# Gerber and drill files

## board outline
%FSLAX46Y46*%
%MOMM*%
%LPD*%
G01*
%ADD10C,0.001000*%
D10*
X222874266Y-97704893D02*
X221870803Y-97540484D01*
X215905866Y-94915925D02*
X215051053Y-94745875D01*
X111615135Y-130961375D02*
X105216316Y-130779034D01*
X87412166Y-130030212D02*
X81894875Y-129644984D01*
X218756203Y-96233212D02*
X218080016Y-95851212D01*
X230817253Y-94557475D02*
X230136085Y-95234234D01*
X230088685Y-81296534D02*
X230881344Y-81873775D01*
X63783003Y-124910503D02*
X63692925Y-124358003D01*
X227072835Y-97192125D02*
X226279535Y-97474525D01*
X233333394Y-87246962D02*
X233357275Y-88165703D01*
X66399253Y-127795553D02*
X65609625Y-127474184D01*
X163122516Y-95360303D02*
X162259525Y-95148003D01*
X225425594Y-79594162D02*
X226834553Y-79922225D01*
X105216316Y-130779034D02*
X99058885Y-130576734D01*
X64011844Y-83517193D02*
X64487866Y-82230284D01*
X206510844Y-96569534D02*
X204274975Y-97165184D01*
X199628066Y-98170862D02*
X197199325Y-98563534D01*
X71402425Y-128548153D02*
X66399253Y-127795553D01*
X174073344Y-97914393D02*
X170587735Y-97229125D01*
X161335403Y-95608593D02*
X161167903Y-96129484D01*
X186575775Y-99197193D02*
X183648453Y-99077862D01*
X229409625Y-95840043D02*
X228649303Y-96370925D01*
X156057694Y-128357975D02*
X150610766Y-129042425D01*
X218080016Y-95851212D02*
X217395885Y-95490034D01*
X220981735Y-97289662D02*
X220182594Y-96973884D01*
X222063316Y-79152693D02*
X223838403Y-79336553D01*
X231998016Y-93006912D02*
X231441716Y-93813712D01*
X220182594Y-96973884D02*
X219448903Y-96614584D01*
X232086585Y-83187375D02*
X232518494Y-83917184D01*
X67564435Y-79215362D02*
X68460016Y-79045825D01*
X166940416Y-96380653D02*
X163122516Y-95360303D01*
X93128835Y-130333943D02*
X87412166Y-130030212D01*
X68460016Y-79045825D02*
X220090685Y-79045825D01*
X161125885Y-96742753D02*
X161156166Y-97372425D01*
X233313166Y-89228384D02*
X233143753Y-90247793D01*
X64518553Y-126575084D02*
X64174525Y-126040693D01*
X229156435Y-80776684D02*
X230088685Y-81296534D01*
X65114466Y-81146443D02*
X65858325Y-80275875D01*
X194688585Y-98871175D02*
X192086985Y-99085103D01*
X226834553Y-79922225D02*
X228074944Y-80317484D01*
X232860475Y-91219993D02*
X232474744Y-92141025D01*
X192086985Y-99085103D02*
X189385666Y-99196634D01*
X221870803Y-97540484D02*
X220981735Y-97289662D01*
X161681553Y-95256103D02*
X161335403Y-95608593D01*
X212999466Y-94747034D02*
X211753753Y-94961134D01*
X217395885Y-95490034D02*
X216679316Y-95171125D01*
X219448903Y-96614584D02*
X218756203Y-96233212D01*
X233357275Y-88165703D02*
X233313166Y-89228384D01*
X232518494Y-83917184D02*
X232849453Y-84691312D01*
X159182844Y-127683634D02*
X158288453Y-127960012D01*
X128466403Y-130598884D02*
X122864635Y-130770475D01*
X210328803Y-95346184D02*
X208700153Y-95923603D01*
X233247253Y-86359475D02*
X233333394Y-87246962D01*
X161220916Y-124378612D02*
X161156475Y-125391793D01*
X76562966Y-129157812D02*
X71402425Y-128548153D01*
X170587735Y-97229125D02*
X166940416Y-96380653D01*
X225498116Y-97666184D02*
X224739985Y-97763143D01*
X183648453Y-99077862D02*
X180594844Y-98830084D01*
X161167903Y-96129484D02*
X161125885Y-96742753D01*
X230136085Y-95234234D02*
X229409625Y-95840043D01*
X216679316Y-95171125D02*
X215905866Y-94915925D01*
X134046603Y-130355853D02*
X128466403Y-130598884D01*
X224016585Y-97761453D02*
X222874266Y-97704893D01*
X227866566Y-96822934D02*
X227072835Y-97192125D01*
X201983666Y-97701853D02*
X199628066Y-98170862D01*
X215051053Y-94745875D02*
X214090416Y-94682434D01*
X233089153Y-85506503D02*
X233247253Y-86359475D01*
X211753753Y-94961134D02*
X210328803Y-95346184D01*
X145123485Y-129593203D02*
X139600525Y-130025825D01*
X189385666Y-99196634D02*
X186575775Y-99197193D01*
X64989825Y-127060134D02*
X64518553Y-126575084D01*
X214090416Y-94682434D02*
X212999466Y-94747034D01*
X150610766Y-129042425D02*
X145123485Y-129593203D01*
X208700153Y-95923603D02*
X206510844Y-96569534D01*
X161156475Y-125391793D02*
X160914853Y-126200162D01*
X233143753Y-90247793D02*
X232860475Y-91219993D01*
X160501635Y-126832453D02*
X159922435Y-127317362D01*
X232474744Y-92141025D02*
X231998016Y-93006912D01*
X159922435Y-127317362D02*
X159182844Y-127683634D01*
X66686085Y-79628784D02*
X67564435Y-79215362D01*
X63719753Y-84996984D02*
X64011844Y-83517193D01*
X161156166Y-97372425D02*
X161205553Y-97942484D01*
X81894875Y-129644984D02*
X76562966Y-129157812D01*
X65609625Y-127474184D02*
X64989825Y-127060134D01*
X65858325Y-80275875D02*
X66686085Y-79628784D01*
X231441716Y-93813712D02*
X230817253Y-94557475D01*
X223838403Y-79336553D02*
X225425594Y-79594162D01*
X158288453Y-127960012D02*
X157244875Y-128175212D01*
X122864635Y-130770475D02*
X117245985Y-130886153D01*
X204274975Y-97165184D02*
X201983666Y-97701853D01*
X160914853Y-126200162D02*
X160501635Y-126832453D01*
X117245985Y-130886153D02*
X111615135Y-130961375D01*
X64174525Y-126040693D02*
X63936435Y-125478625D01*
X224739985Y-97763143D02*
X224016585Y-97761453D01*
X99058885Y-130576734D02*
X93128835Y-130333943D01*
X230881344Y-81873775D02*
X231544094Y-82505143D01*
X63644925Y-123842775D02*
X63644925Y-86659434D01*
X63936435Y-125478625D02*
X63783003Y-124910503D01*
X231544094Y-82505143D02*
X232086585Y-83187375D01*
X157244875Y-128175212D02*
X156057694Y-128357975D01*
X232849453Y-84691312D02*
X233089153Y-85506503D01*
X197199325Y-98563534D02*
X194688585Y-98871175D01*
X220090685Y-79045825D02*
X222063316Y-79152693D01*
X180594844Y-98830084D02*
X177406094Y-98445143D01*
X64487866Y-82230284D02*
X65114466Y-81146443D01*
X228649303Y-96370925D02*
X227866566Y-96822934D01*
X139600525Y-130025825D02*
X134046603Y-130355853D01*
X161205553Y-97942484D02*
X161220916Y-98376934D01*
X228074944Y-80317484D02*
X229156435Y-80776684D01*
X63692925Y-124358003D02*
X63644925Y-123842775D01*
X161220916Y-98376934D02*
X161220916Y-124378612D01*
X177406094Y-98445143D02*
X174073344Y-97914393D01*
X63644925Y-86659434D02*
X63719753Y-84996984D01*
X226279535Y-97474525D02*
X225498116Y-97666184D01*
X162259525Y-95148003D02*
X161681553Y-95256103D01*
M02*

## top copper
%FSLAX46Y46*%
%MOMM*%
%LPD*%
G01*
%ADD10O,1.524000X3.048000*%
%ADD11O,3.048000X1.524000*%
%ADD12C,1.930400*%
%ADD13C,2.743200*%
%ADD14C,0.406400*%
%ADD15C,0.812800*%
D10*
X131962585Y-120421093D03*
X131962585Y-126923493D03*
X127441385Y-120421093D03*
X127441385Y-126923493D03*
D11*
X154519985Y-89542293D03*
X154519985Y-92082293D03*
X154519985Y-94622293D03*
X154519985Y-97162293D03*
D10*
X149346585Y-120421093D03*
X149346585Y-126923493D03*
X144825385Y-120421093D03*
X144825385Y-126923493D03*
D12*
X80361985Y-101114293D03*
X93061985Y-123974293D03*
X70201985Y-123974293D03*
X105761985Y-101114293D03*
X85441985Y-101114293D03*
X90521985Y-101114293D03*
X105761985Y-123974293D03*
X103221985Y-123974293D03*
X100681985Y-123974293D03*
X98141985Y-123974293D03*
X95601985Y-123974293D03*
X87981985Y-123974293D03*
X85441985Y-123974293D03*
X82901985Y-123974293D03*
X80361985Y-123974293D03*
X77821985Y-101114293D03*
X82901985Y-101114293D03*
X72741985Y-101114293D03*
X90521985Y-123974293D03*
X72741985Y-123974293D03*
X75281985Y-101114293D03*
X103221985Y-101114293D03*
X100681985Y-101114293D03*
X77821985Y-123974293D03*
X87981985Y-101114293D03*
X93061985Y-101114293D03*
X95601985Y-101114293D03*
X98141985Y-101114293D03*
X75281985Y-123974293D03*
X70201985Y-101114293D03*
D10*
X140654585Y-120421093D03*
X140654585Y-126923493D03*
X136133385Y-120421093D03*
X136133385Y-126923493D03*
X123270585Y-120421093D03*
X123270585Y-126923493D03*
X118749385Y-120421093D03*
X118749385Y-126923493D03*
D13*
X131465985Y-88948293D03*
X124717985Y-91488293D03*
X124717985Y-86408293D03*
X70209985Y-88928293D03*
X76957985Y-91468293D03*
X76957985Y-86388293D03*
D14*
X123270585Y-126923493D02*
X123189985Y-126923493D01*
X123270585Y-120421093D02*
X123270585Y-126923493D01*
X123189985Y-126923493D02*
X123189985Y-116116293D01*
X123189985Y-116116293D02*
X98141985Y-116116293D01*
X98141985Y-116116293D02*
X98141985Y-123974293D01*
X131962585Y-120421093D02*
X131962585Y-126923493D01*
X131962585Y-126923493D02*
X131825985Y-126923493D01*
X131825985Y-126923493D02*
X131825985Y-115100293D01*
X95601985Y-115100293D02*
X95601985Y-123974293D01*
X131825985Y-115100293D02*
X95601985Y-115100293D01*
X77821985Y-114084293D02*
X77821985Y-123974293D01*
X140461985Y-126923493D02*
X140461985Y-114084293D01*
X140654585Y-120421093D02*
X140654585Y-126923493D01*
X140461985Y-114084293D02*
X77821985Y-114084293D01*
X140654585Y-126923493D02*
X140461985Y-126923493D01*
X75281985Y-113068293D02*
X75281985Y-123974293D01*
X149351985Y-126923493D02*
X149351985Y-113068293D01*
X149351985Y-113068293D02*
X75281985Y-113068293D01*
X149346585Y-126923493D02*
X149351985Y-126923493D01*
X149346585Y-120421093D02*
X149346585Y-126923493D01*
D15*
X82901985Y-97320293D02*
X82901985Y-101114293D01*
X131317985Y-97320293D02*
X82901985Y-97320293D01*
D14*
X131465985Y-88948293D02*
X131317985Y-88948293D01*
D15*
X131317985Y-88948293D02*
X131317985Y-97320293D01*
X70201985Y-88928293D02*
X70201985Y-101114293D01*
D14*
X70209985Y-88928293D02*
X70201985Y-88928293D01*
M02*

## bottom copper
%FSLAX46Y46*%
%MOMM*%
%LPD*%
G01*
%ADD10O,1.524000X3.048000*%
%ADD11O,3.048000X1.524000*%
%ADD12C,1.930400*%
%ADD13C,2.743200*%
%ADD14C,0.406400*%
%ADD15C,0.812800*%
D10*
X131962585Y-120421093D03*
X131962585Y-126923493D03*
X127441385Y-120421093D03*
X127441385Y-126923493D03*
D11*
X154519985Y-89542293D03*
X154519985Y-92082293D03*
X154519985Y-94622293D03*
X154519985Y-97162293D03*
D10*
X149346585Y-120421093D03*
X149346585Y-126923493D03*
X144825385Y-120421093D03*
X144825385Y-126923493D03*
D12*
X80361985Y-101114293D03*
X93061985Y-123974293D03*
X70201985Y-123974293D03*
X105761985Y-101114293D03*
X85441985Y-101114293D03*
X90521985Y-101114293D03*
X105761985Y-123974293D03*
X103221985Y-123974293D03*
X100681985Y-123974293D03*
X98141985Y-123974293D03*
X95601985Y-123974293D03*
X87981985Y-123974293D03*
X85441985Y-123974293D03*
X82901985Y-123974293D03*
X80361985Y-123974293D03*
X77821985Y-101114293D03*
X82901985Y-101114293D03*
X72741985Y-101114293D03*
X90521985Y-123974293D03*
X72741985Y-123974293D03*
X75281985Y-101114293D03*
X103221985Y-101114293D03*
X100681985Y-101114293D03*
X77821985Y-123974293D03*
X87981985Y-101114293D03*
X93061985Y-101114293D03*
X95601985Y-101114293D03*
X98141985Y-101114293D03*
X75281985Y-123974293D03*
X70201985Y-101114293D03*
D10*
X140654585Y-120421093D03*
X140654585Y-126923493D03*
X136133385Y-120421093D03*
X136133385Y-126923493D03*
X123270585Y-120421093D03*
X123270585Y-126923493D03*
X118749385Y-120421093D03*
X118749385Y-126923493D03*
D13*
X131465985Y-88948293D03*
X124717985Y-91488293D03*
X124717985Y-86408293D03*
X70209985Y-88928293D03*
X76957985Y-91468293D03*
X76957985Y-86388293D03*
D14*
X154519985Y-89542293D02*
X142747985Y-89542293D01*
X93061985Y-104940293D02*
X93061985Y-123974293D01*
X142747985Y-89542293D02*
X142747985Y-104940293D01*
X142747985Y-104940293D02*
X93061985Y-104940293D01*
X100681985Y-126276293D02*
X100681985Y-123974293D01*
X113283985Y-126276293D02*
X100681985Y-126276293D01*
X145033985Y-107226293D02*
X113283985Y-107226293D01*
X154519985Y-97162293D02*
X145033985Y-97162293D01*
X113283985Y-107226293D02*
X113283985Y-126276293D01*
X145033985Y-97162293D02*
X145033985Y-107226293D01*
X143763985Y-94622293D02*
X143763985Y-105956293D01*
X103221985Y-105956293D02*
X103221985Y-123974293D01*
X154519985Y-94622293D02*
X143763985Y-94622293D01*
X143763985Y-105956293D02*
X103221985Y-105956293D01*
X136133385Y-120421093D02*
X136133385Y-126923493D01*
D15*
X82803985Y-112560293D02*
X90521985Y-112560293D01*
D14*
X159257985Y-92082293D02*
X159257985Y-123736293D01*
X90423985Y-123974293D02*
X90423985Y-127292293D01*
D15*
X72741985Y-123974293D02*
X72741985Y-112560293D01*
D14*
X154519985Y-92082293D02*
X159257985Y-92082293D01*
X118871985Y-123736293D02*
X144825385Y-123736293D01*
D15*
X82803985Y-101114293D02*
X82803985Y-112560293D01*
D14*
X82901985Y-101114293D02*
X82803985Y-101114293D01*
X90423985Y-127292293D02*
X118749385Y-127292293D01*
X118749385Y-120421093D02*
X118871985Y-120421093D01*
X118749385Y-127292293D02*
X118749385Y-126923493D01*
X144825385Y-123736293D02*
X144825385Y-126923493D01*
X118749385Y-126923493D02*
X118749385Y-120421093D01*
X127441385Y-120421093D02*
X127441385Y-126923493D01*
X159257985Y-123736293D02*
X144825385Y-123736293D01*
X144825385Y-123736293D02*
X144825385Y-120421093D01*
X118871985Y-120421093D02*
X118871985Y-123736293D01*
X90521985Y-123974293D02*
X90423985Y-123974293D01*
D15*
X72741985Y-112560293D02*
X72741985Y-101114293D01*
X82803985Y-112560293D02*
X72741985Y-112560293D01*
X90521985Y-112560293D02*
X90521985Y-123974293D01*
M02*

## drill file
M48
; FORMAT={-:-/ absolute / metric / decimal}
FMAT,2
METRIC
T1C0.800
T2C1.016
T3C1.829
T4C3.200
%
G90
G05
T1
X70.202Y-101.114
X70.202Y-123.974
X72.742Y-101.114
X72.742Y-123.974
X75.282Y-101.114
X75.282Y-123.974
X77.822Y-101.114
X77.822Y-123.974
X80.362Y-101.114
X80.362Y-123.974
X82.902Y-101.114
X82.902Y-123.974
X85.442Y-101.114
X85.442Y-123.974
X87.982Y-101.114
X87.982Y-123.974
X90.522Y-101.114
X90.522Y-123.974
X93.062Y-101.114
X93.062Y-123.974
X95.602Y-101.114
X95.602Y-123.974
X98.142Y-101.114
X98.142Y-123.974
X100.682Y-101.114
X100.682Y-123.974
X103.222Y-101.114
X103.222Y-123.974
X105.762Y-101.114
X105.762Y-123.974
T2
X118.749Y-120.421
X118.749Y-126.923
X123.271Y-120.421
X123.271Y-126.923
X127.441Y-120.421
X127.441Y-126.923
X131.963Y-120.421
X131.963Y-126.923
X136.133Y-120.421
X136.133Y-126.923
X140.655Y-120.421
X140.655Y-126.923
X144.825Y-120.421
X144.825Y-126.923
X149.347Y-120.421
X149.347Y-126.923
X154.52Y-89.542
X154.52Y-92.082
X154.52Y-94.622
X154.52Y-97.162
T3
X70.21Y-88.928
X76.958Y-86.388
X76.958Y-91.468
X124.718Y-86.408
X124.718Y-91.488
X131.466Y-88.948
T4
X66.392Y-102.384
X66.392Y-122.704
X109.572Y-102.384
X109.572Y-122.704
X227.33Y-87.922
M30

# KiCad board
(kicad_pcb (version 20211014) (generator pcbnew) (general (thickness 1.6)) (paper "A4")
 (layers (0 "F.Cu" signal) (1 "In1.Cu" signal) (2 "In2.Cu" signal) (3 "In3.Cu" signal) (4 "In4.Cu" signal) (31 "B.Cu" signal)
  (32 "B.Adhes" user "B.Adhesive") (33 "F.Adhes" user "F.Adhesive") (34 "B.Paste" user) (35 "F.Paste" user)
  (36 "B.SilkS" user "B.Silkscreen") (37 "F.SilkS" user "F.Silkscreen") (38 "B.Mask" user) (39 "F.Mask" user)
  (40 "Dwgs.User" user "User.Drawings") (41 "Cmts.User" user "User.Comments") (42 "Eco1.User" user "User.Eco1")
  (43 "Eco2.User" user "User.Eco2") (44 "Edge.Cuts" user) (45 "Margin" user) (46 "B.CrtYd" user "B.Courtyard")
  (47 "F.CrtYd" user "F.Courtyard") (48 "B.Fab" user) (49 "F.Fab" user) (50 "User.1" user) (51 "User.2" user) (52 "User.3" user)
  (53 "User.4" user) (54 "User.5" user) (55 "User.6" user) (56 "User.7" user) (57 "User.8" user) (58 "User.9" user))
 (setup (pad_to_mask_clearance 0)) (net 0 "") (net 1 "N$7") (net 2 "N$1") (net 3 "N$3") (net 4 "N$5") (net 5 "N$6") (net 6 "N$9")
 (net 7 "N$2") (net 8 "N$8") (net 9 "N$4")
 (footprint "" (layer "F.Cu") (at 227.329985 87.922293)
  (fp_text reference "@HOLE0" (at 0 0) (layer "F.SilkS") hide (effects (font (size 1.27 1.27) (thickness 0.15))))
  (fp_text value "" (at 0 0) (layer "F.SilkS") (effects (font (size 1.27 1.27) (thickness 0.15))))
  (pad "" np_thru_hole circle (at 0 0) (size 3.2 3.2) (drill 3.2) (layers *.Cu *.Mask)))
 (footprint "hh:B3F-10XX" (layer "F.Cu") (at 129.701985 123.672293 -90)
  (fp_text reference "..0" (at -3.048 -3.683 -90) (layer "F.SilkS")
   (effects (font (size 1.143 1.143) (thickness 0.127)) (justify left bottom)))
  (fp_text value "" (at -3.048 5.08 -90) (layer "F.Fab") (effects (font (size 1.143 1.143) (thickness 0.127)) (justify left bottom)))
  (pad "1" thru_hole oval (at -3.2512 -2.2606 270) (size 3.048 1.524) (drill 1.016) (layers *.Cu *.Mask) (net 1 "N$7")
   (solder_mask_margin 0.0635))
  (pad "2" thru_hole oval (at 3.2512 -2.2606 270) (size 3.048 1.524) (drill 1.016) (layers *.Cu *.Mask) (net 1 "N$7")
   (solder_mask_margin 0.0635))
  (pad "3" thru_hole oval (at -3.2512 2.2606 270) (size 3.048 1.524) (drill 1.016) (layers *.Cu *.Mask) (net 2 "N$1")
   (solder_mask_margin 0.0635))
  (pad "4" thru_hole oval (at 3.2512 2.2606 270) (size 3.048 1.524) (drill 1.016) (layers *.Cu *.Mask) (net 2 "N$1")
   (solder_mask_margin 0.0635)))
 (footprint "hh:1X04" (layer "F.Cu") (at 154.519985 93.352293 -90)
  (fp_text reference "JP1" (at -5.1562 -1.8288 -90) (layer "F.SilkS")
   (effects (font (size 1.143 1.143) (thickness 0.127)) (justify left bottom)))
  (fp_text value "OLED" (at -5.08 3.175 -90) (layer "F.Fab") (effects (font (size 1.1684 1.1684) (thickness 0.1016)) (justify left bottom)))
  (pad "1" thru_hole oval (at -3.81 0) (size 3.048 1.524) (drill 1.016) (layers *.Cu *.Mask) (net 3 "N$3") (solder_mask_margin 0.0635))
  (pad "2" thru_hole oval (at -1.27 0) (size 3.048 1.524) (drill 1.016) (layers *.Cu *.Mask) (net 2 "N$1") (solder_mask_margin 0.0635))
  (pad "3" thru_hole oval (at 1.27 0) (size 3.048 1.524) (drill 1.016) (layers *.Cu *.Mask) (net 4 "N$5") (solder_mask_margin 0.0635))
  (pad "4" thru_hole oval (at 3.81 0) (size 3.048 1.524) (drill 1.016) (layers *.Cu *.Mask) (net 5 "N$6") (solder_mask_margin 0.0635)))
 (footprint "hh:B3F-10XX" (layer "F.Cu") (at 147.085985 123.672293 -90)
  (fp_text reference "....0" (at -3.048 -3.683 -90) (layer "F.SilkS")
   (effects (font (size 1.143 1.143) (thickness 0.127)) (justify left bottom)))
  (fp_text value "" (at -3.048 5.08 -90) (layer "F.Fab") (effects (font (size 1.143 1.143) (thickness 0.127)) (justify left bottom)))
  (pad "1" thru_hole oval (at -3.2512 -2.2606 270) (size 3.048 1.524) (drill 1.016) (layers *.Cu *.Mask) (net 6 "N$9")
   (solder_mask_margin 0.0635))
  (pad "2" thru_hole oval (at 3.2512 -2.2606 270) (size 3.048 1.524) (drill 1.016) (layers *.Cu *.Mask) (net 6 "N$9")
   (solder_mask_margin 0.0635))
  (pad "3" thru_hole oval (at -3.2512 2.2606 270) (size 3.048 1.524) (drill 1.016) (layers *.Cu *.Mask) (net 2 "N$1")
   (solder_mask_margin 0.0635))
  (pad "4" thru_hole oval (at 3.2512 2.2606 270) (size 3.048 1.524) (drill 1.016) (layers *.Cu *.Mask) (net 2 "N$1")
   (solder_mask_margin 0.0635)))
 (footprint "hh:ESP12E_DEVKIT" (layer "F.Cu") (at 87.981985 112.544293 -90)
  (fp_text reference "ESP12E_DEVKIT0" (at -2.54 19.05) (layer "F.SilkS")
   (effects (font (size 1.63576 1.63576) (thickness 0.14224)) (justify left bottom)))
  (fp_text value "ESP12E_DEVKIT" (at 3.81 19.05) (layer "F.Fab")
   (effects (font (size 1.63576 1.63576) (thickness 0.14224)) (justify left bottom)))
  (pad "" np_thru_hole circle (at -10.16 -21.59 270) (size 3.2 3.2) (drill 3.2) (layers *.Cu *.Mask))
  (pad "" np_thru_hole circle (at 10.16 21.59 270) (size 3.2 3.2) (drill 3.2) (layers *.Cu *.Mask))
  (pad "" np_thru_hole circle (at -10.16 21.59 270) (size 3.2 3.2) (drill 3.2) (layers *.Cu *.Mask))
  (pad "" np_thru_hole circle (at 10.16 -21.59 270) (size 3.2 3.2) (drill 3.2) (layers *.Cu *.Mask))
  (pad "3V3@0" thru_hole circle (at -11.43 7.62 270) (size 1.9304 1.9304) (drill 0.8) (layers *.Cu *.Mask) (solder_mask_margin 0.0635))
  (pad "3V3@1" thru_hole circle (at 11.43 -5.08 270) (size 1.9304 1.9304) (drill 0.8) (layers *.Cu *.Mask) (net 3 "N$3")
   (solder_mask_margin 0.0635))
  (pad "3V3@2" thru_hole circle (at 11.43 17.78 270) (size 1.9304 1.9304) (drill 0.8) (layers *.Cu *.Mask) (solder_mask_margin 0.0635))
  (pad "AD0" thru_hole circle (at -11.43 -17.78 270) (size 1.9304 1.9304) (drill 0.8) (layers *.Cu *.Mask) (solder_mask_margin 0.0635))
  (pad "CLK" thru_hole circle (at -11.43 2.54 270) (size 1.9304 1.9304) (drill 0.8) (layers *.Cu *.Mask) (solder_mask_margin 0.0635))
  (pad "CMD" thru_hole circle (at -11.43 -2.54 270) (size 1.9304 1.9304) (drill 0.8) (layers *.Cu *.Mask) (solder_mask_margin 0.0635))
  (pad "D0" thru_hole circle (at 11.43 -17.78 270) (size 1.9304 1.9304) (drill 0.8) (layers *.Cu *.Mask) (solder_mask_margin 0.0635))
  (pad "D1" thru_hole circle (at 11.43 -15.24 270) (size 1.9304 1.9304) (drill 0.8) (layers *.Cu *.Mask) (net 4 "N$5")
   (solder_mask_margin 0.0635))
  (pad "D2" thru_hole circle (at 11.43 -12.7 270) (size 1.9304 1.9304) (drill 0.8) (layers *.Cu *.Mask) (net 5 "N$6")
   (solder_mask_margin 0.0635))
  (pad "D3" thru_hole circle (at 11.43 -10.16 270) (size 1.9304 1.9304) (drill 0.8) (layers *.Cu *.Mask) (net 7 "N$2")
   (solder_mask_margin 0.0635))
  (pad "D4" thru_hole circle (at 11.43 -7.62 270) (size 1.9304 1.9304) (drill 0.8) (layers *.Cu *.Mask) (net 1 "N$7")
   (solder_mask_margin 0.0635))
  (pad "D5" thru_hole circle (at 11.43 0 270) (size 1.9304 1.9304) (drill 0.8) (layers *.Cu *.Mask) (solder_mask_margin 0.0635))
  (pad "D6" thru_hole circle (at 11.43 2.54 270) (size 1.9304 1.9304) (drill 0.8) (layers *.Cu *.Mask) (solder_mask_margin 0.0635))
  (pad "D7" thru_hole circle (at 11.43 5.08 270) (size 1.9304 1.9304) (drill 0.8) (layers *.Cu *.Mask) (solder_mask_margin 0.0635))
  (pad "D8" thru_hole circle (at 11.43 7.62 270) (size 1.9304 1.9304) (drill 0.8) (layers *.Cu *.Mask) (solder_mask_margin 0.0635))
  (pad "EN" thru_hole circle (at -11.43 10.16 270) (size 1.9304 1.9304) (drill 0.8) (layers *.Cu *.Mask) (solder_mask_margin 0.0635))
  (pad "GND@0" thru_hole circle (at -11.43 5.08 270) (size 1.9304 1.9304) (drill 0.8) (layers *.Cu *.Mask) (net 2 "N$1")
   (solder_mask_margin 0.0635))
  (pad "GND@1" thru_hole circle (at -11.43 15.24 270) (size 1.9304 1.9304) (drill 0.8) (layers *.Cu *.Mask) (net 2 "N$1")
   (solder_mask_margin 0.0635))
  (pad "GND@2" thru_hole circle (at 11.43 -2.54 270) (size 1.9304 1.9304) (drill 0.8) (layers *.Cu *.Mask) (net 2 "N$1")
   (solder_mask_margin 0.0635))
  (pad "GND@3" thru_hole circle (at 11.43 15.24 270) (size 1.9304 1.9304) (drill 0.8) (layers *.Cu *.Mask) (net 2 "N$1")
   (solder_mask_margin 0.0635))
  (pad "RST" thru_hole circle (at -11.43 12.7 270) (size 1.9304 1.9304) (drill 0.8) (layers *.Cu *.Mask) (solder_mask_margin 0.0635))
  (pad "RSV@0" thru_hole circle (at -11.43 -15.24 270) (size 1.9304 1.9304) (drill 0.8) (layers *.Cu *.Mask) (solder_mask_margin 0.0635))
  (pad "RSV@1" thru_hole circle (at -11.43 -12.7 270) (size 1.9304 1.9304) (drill 0.8) (layers *.Cu *.Mask) (solder_mask_margin 0.0635))
  (pad "RX" thru_hole circle (at 11.43 10.16 270) (size 1.9304 1.9304) (drill 0.8) (layers *.Cu *.Mask) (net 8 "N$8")
   (solder_mask_margin 0.0635))
  (pad "SD0" thru_hole circle (at -11.43 0 270) (size 1.9304 1.9304) (drill 0.8) (layers *.Cu *.Mask) (solder_mask_margin 0.0635))
  (pad "SD1" thru_hole circle (at -11.43 -5.08 270) (size 1.9304 1.9304) (drill 0.8) (layers *.Cu *.Mask) (solder_mask_margin 0.0635))
  (pad "SD2" thru_hole circle (at -11.43 -7.62 270) (size 1.9304 1.9304) (drill 0.8) (layers *.Cu *.Mask) (solder_mask_margin 0.0635))
  (pad "SD3" thru_hole circle (at -11.43 -10.16 270) (size 1.9304 1.9304) (drill 0.8) (layers *.Cu *.Mask) (solder_mask_margin 0.0635))
  (pad "TX" thru_hole circle (at 11.43 12.7 270) (size 1.9304 1.9304) (drill 0.8) (layers *.Cu *.Mask) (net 6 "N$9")
   (solder_mask_margin 0.0635))
  (pad "VIN" thru_hole circle (at -11.43 17.78 270) (size 1.9304 1.9304) (drill 0.8) (layers *.Cu *.Mask) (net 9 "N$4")
   (solder_mask_margin 0.0635)))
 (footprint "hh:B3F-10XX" (layer "F.Cu") (at 138.393985 123.672293 -90)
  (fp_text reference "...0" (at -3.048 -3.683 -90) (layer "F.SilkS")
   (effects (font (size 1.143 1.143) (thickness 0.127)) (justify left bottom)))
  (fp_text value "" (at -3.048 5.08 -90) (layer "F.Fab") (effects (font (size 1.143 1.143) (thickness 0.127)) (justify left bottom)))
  (pad "1" thru_hole oval (at -3.2512 -2.2606 270) (size 3.048 1.524) (drill 1.016) (layers *.Cu *.Mask) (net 8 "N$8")
   (solder_mask_margin 0.0635))
  (pad "2" thru_hole oval (at 3.2512 -2.2606 270) (size 3.048 1.524) (drill 1.016) (layers *.Cu *.Mask) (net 8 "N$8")
   (solder_mask_margin 0.0635))
  (pad "3" thru_hole oval (at -3.2512 2.2606 270) (size 3.048 1.524) (drill 1.016) (layers *.Cu *.Mask) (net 2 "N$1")
   (solder_mask_margin 0.0635))
  (pad "4" thru_hole oval (at 3.2512 2.2606 270) (size 3.048 1.524) (drill 1.016) (layers *.Cu *.Mask) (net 2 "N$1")
   (solder_mask_margin 0.0635)))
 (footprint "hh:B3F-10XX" (layer "F.Cu") (at 121.009985 123.672293 -90)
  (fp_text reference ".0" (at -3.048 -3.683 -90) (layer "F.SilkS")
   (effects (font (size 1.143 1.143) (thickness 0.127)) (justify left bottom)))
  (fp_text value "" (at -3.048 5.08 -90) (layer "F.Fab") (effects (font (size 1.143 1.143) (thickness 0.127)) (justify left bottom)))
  (pad "1" thru_hole oval (at -3.2512 -2.2606 270) (size 3.048 1.524) (drill 1.016) (layers *.Cu *.Mask) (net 7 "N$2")
   (solder_mask_margin 0.0635))
  (pad "2" thru_hole oval (at 3.2512 -2.2606 270) (size 3.048 1.524) (drill 1.016) (layers *.Cu *.Mask) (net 7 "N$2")
   (solder_mask_margin 0.0635))
  (pad "3" thru_hole oval (at -3.2512 2.2606 270) (size 3.048 1.524) (drill 1.016) (layers *.Cu *.Mask) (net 2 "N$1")
   (solder_mask_margin 0.0635))
  (pad "4" thru_hole oval (at 3.2512 2.2606 270) (size 3.048 1.524) (drill 1.016) (layers *.Cu *.Mask) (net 2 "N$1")
   (solder_mask_margin 0.0635)))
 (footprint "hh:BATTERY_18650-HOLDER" (layer "B.Cu") (at 100.837985 88.938293)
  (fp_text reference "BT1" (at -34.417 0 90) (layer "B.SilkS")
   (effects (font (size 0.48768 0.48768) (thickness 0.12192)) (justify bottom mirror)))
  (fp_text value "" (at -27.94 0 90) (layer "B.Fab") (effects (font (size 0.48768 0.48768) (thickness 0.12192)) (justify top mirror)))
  (pad "GND@1" thru_hole circle (at 30.628 0.01 180) (size 2.7432 2.7432) (drill 1.8288) (layers *.Cu *.Mask) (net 2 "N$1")
   (solder_mask_margin 0.0635))
  (pad "GND@2" thru_hole circle (at 23.88 2.55 90) (size 2.7432 2.7432) (drill 1.8288) (layers *.Cu *.Mask) (solder_mask_margin 0.0635))
  (pad "GND@3" thru_hole circle (at 23.88 -2.53 90) (size 2.7432 2.7432) (drill 1.8288) (layers *.Cu *.Mask) (solder_mask_margin 0.0635))
  (pad "PWR@1" thru_hole circle (at -30.628 -0.01) (size 2.7432 2.7432) (drill 1.8288) (layers *.Cu *.Mask) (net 9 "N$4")
   (solder_mask_margin 0.0635))
  (pad "PWR@2" thru_hole circle (at -23.88 2.53 270) (size 2.7432 2.7432) (drill 1.8288) (layers *.Cu *.Mask) (solder_mask_margin 0.0635))
  (pad "PWR@3" thru_hole circle (at -23.88 -2.55 270) (size 2.7432 2.7432) (drill 1.8288) (layers *.Cu *.Mask) (solder_mask_margin 0.0635)))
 (gr_line (start 222.874266 97.704893) (end 221.870803 97.540484) (layer "Edge.Cuts") (width 0.001))
 (gr_line (start 215.905866 94.915925) (end 215.051053 94.745875) (layer "Edge.Cuts") (width 0.001))
 (gr_line (start 111.615135 130.961375) (end 105.216316 130.779034) (layer "Edge.Cuts") (width 0.001))
 (gr_line (start 87.412166 130.030212) (end 81.894875 129.644984) (layer "Edge.Cuts") (width 0.001))
 (gr_line (start 218.756203 96.233212) (end 218.080016 95.851212) (layer "Edge.Cuts") (width 0.001))
 (gr_line (start 230.817253 94.557475) (end 230.136085 95.234234) (layer "Edge.Cuts") (width 0.001))
 (gr_line (start 230.088685 81.296534) (end 230.881344 81.873775) (layer "Edge.Cuts") (width 0.001))
 (gr_line (start 63.783003 124.910503) (end 63.692925 124.358003) (layer "Edge.Cuts") (width 0.001))
 (gr_line (start 227.072835 97.192125) (end 226.279535 97.474525) (layer "Edge.Cuts") (width 0.001))
 (gr_line (start 233.333394 87.246962) (end 233.357275 88.165703) (layer "Edge.Cuts") (width 0.001))
 (gr_line (start 66.399253 127.795553) (end 65.609625 127.474184) (layer "Edge.Cuts") (width 0.001))
 (gr_line (start 163.122516 95.360303) (end 162.259525 95.148003) (layer "Edge.Cuts") (width 0.001))
 (gr_line (start 225.425594 79.594162) (end 226.834553 79.922225) (layer "Edge.Cuts") (width 0.001))
 (gr_line (start 105.216316 130.779034) (end 99.058885 130.576734) (layer "Edge.Cuts") (width 0.001))
 (gr_line (start 64.011844 83.517193) (end 64.487866 82.230284) (layer "Edge.Cuts") (width 0.001))
 (gr_line (start 206.510844 96.569534) (end 204.274975 97.165184) (layer "Edge.Cuts") (width 0.001))
 (gr_line (start 199.628066 98.170862) (end 197.199325 98.563534) (layer "Edge.Cuts") (width 0.001))
 (gr_line (start 71.402425 128.548153) (end 66.399253 127.795553) (layer "Edge.Cuts") (width 0.001))
 (gr_line (start 174.073344 97.914393) (end 170.587735 97.229125) (layer "Edge.Cuts") (width 0.001))
 (gr_line (start 161.335403 95.608593) (end 161.167903 96.129484) (layer "Edge.Cuts") (width 0.001))
 (gr_line (start 186.575775 99.197193) (end 183.648453 99.077862) (layer "Edge.Cuts") (width 0.001))
 (gr_line (start 229.409625 95.840043) (end 228.649303 96.370925) (layer "Edge.Cuts") (width 0.001))
 (gr_line (start 156.057694 128.357975) (end 150.610766 129.042425) (layer "Edge.Cuts") (width 0.001))
 (gr_line (start 218.080016 95.851212) (end 217.395885 95.490034) (layer "Edge.Cuts") (width 0.001))
 (gr_line (start 220.981735 97.289662) (end 220.182594 96.973884) (layer "Edge.Cuts") (width 0.001))
 (gr_line (start 222.063316 79.152693) (end 223.838403 79.336553) (layer "Edge.Cuts") (width 0.001))
 (gr_line (start 231.998016 93.006912) (end 231.441716 93.813712) (layer "Edge.Cuts") (width 0.001))
 (gr_line (start 220.182594 96.973884) (end 219.448903 96.614584) (layer "Edge.Cuts") (width 0.001))
 (gr_line (start 232.086585 83.187375) (end 232.518494 83.917184) (layer "Edge.Cuts") (width 0.001))
 (gr_line (start 67.564435 79.215362) (end 68.460016 79.045825) (layer "Edge.Cuts") (width 0.001))
 (gr_line (start 166.940416 96.380653) (end 163.122516 95.360303) (layer "Edge.Cuts") (width 0.001))
 (gr_line (start 93.128835 130.333943) (end 87.412166 130.030212) (layer "Edge.Cuts") (width 0.001))
 (gr_line (start 68.460016 79.045825) (end 220.090685 79.045825) (layer "Edge.Cuts") (width 0.001))
 (gr_line (start 161.125885 96.742753) (end 161.156166 97.372425) (layer "Edge.Cuts") (width 0.001))
 (gr_line (start 233.313166 89.228384) (end 233.143753 90.247793) (layer "Edge.Cuts") (width 0.001))
 (gr_line (start 64.518553 126.575084) (end 64.174525 126.040693) (layer "Edge.Cuts") (width 0.001))
 (gr_line (start 229.156435 80.776684) (end 230.088685 81.296534) (layer "Edge.Cuts") (width 0.001))
 (gr_line (start 65.114466 81.146443) (end 65.858325 80.275875) (layer "Edge.Cuts") (width 0.001))
 (gr_line (start 194.688585 98.871175) (end 192.086985 99.085103) (layer "Edge.Cuts") (width 0.001))
 (gr_line (start 226.834553 79.922225) (end 228.074944 80.317484) (layer "Edge.Cuts") (width 0.001))
 (gr_line (start 232.860475 91.219993) (end 232.474744 92.141025) (layer "Edge.Cuts") (width 0.001))
 (gr_line (start 192.086985 99.085103) (end 189.385666 99.196634) (layer "Edge.Cuts") (width 0.001))
 (gr_line (start 221.870803 97.540484) (end 220.981735 97.289662) (layer "Edge.Cuts") (width 0.001))
 (gr_line (start 161.681553 95.256103) (end 161.335403 95.608593) (layer "Edge.Cuts") (width 0.001))
 (gr_line (start 212.999466 94.747034) (end 211.753753 94.961134) (layer "Edge.Cuts") (width 0.001))
 (gr_line (start 217.395885 95.490034) (end 216.679316 95.171125) (layer "Edge.Cuts") (width 0.001))
 (gr_line (start 219.448903 96.614584) (end 218.756203 96.233212) (layer "Edge.Cuts") (width 0.001))
 (gr_line (start 233.357275 88.165703) (end 233.313166 89.228384) (layer "Edge.Cuts") (width 0.001))
 (gr_line (start 232.518494 83.917184) (end 232.849453 84.691312) (layer "Edge.Cuts") (width 0.001))
 (gr_line (start 159.182844 127.683634) (end 158.288453 127.960012) (layer "Edge.Cuts") (width 0.001))
 (gr_line (start 128.466403 130.598884) (end 122.864635 130.770475) (layer "Edge.Cuts") (width 0.001))
 (gr_line (start 210.328803 95.346184) (end 208.700153 95.923603) (layer "Edge.Cuts") (width 0.001))
 (gr_line (start 233.247253 86.359475) (end 233.333394 87.246962) (layer "Edge.Cuts") (width 0.001))
 (gr_line (start 161.220916 124.378612) (end 161.156475 125.391793) (layer "Edge.Cuts") (width 0.001))
 (gr_line (start 76.562966 129.157812) (end 71.402425 128.548153) (layer "Edge.Cuts") (width 0.001))
 (gr_line (start 170.587735 97.229125) (end 166.940416 96.380653) (layer "Edge.Cuts") (width 0.001))
 (gr_line (start 225.498116 97.666184) (end 224.739985 97.763143) (layer "Edge.Cuts") (width 0.001))
 (gr_line (start 183.648453 99.077862) (end 180.594844 98.830084) (layer "Edge.Cuts") (width 0.001))
 (gr_line (start 161.167903 96.129484) (end 161.125885 96.742753) (layer "Edge.Cuts") (width 0.001))
 (gr_line (start 230.136085 95.234234) (end 229.409625 95.840043) (layer "Edge.Cuts") (width 0.001))
 (gr_line (start 216.679316 95.171125) (end 215.905866 94.915925) (layer "Edge.Cuts") (width 0.001))
 (gr_line (start 134.046603 130.355853) (end 128.466403 130.598884) (layer "Edge.Cuts") (width 0.001))
 (gr_line (start 224.016585 97.761453) (end 222.874266 97.704893) (layer "Edge.Cuts") (width 0.001))
 (gr_line (start 227.866566 96.822934) (end 227.072835 97.192125) (layer "Edge.Cuts") (width 0.001))
 (gr_line (start 201.983666 97.701853) (end 199.628066 98.170862) (layer "Edge.Cuts") (width 0.001))
 (gr_line (start 215.051053 94.745875) (end 214.090416 94.682434) (layer "Edge.Cuts") (width 0.001))
 (gr_line (start 233.089153 85.506503) (end 233.247253 86.359475) (layer "Edge.Cuts") (width 0.001))
 (gr_line (start 211.753753 94.961134) (end 210.328803 95.346184) (layer "Edge.Cuts") (width 0.001))
 (gr_line (start 145.123485 129.593203) (end 139.600525 130.025825) (layer "Edge.Cuts") (width 0.001))
 (gr_line (start 189.385666 99.196634) (end 186.575775 99.197193) (layer "Edge.Cuts") (width 0.001))
 (gr_line (start 64.989825 127.060134) (end 64.518553 126.575084) (layer "Edge.Cuts") (width 0.001))
 (gr_line (start 214.090416 94.682434) (end 212.999466 94.747034) (layer "Edge.Cuts") (width 0.001))
 (gr_line (start 150.610766 129.042425) (end 145.123485 129.593203) (layer "Edge.Cuts") (width 0.001))
 (gr_line (start 208.700153 95.923603) (end 206.510844 96.569534) (layer "Edge.Cuts") (width 0.001))
 (gr_line (start 161.156475 125.391793) (end 160.914853 126.200162) (layer "Edge.Cuts") (width 0.001))
 (gr_line (start 233.143753 90.247793) (end 232.860475 91.219993) (layer "Edge.Cuts") (width 0.001))
 (gr_line (start 160.501635 126.832453) (end 159.922435 127.317362) (layer "Edge.Cuts") (width 0.001))
 (gr_line (start 232.474744 92.141025) (end 231.998016 93.006912) (layer "Edge.Cuts") (width 0.001))
 (gr_line (start 159.922435 127.317362) (end 159.182844 127.683634) (layer "Edge.Cuts") (width 0.001))
 (gr_line (start 66.686085 79.628784) (end 67.564435 79.215362) (layer "Edge.Cuts") (width 0.001))
 (gr_line (start 63.719753 84.996984) (end 64.011844 83.517193) (layer "Edge.Cuts") (width 0.001))
 (gr_line (start 161.156166 97.372425) (end 161.205553 97.942484) (layer "Edge.Cuts") (width 0.001))
 (gr_line (start 81.894875 129.644984) (end 76.562966 129.157812) (layer "Edge.Cuts") (width 0.001))
 (gr_line (start 65.609625 127.474184) (end 64.989825 127.060134) (layer "Edge.Cuts") (width 0.001))
 (gr_line (start 65.858325 80.275875) (end 66.686085 79.628784) (layer "Edge.Cuts") (width 0.001))
 (gr_line (start 231.441716 93.813712) (end 230.817253 94.557475) (layer "Edge.Cuts") (width 0.001))
 (gr_line (start 223.838403 79.336553) (end 225.425594 79.594162) (layer "Edge.Cuts") (width 0.001))
 (gr_line (start 158.288453 127.960012) (end 157.244875 128.175212) (layer "Edge.Cuts") (width 0.001))
 (gr_line (start 122.864635 130.770475) (end 117.245985 130.886153) (layer "Edge.Cuts") (width 0.001))
 (gr_line (start 204.274975 97.165184) (end 201.983666 97.701853) (layer "Edge.Cuts") (width 0.001))
 (gr_line (start 160.914853 126.200162) (end 160.501635 126.832453) (layer "Edge.Cuts") (width 0.001))
 (gr_line (start 117.245985 130.886153) (end 111.615135 130.961375) (layer "Edge.Cuts") (width 0.001))
 (gr_line (start 64.174525 126.040693) (end 63.936435 125.478625) (layer "Edge.Cuts") (width 0.001))
 (gr_line (start 224.739985 97.763143) (end 224.016585 97.761453) (layer "Edge.Cuts") (width 0.001))
 (gr_line (start 99.058885 130.576734) (end 93.128835 130.333943) (layer "Edge.Cuts") (width 0.001))
 (gr_line (start 230.881344 81.873775) (end 231.544094 82.505143) (layer "Edge.Cuts") (width 0.001))
 (gr_line (start 63.644925 123.842775) (end 63.644925 86.659434) (layer "Edge.Cuts") (width 0.001))
 (gr_line (start 63.936435 125.478625) (end 63.783003 124.910503) (layer "Edge.Cuts") (width 0.001))
 (gr_line (start 231.544094 82.505143) (end 232.086585 83.187375) (layer "Edge.Cuts") (width 0.001))
 (gr_line (start 157.244875 128.175212) (end 156.057694 128.357975) (layer "Edge.Cuts") (width 0.001))
 (gr_line (start 232.849453 84.691312) (end 233.089153 85.506503) (layer "Edge.Cuts") (width 0.001))
 (gr_line (start 197.199325 98.563534) (end 194.688585 98.871175) (layer "Edge.Cuts") (width 0.001))
 (gr_line (start 220.090685 79.045825) (end 222.063316 79.152693) (layer "Edge.Cuts") (width 0.001))
 (gr_line (start 180.594844 98.830084) (end 177.406094 98.445143) (layer "Edge.Cuts") (width 0.001))
 (gr_line (start 64.487866 82.230284) (end 65.114466 81.146443) (layer "Edge.Cuts") (width 0.001))
 (gr_line (start 228.649303 96.370925) (end 227.866566 96.822934) (layer "Edge.Cuts") (width 0.001))
 (gr_line (start 139.600525 130.025825) (end 134.046603 130.355853) (layer "Edge.Cuts") (width 0.001))
 (gr_line (start 161.205553 97.942484) (end 161.220916 98.376934) (layer "Edge.Cuts") (width 0.001))
 (gr_line (start 228.074944 80.317484) (end 229.156435 80.776684) (layer "Edge.Cuts") (width 0.001))
 (gr_line (start 63.692925 124.358003) (end 63.644925 123.842775) (layer "Edge.Cuts") (width 0.001))
 (gr_line (start 161.220916 98.376934) (end 161.220916 124.378612) (layer "Edge.Cuts") (width 0.001))
 (gr_line (start 177.406094 98.445143) (end 174.073344 97.914393) (layer "Edge.Cuts") (width 0.001))
 (gr_line (start 63.644925 86.659434) (end 63.719753 84.996984) (layer "Edge.Cuts") (width 0.001))
 (gr_line (start 226.279535 97.474525) (end 225.498116 97.666184) (layer "Edge.Cuts") (width 0.001))
 (gr_line (start 162.259525 95.148003) (end 161.681553 95.256103) (layer "Edge.Cuts") (width 0.001))
 (segment (start 154.519985 89.542293) (end 142.747985 89.542293) (width 0.4064) (layer "B.Cu") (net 3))
 (segment (start 93.061985 104.940293) (end 93.061985 123.974293) (width 0.4064) (layer "B.Cu") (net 3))
 (segment (start 142.747985 89.542293) (end 142.747985 104.940293) (width 0.4064) (layer "B.Cu") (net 3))
 (segment (start 142.747985 104.940293) (end 93.061985 104.940293) (width 0.4064) (layer "B.Cu") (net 3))
 (segment (start 100.681985 126.276293) (end 100.681985 123.974293) (width 0.4064) (layer "B.Cu") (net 5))
 (segment (start 113.283985 126.276293) (end 100.681985 126.276293) (width 0.4064) (layer "B.Cu") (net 5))
 (segment (start 145.033985 107.226293) (end 113.283985 107.226293) (width 0.4064) (layer "B.Cu") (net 5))
 (segment (start 154.519985 97.162293) (end 145.033985 97.162293) (width 0.4064) (layer "B.Cu") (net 5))
 (segment (start 113.283985 107.226293) (end 113.283985 126.276293) (width 0.4064) (layer "B.Cu") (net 5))
 (segment (start 145.033985 97.162293) (end 145.033985 107.226293) (width 0.4064) (layer "B.Cu") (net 5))
 (segment (start 143.763985 94.622293) (end 143.763985 105.956293) (width 0.4064) (layer "B.Cu") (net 4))
 (segment (start 103.221985 105.956293) (end 103.221985 123.974293) (width 0.4064) (layer "B.Cu") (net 4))
 (segment (start 154.519985 94.622293) (end 143.763985 94.622293) (width 0.4064) (layer "B.Cu") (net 4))
 (segment (start 143.763985 105.956293) (end 103.221985 105.956293) (width 0.4064) (layer "B.Cu") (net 4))
 (segment (start 123.270585 126.923493) (end 123.189985 126.923493) (width 0.4064) (layer "F.Cu") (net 7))
 (segment (start 123.270585 120.421093) (end 123.270585 126.923493) (width 0.4064) (layer "F.Cu") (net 7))
 (segment (start 123.189985 126.923493) (end 123.189985 116.116293) (width 0.4064) (layer "F.Cu") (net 7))
 (segment (start 123.189985 116.116293) (end 98.141985 116.116293) (width 0.4064) (layer "F.Cu") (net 7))
 (segment (start 98.141985 116.116293) (end 98.141985 123.974293) (width 0.4064) (layer "F.Cu") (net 7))
 (segment (start 131.962585 120.421093) (end 131.962585 126.923493) (width 0.4064) (layer "F.Cu") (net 1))
 (segment (start 131.962585 126.923493) (end 131.825985 126.923493) (width 0.4064) (layer "F.Cu") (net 1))
 (segment (start 131.825985 126.923493) (end 131.825985 115.100293) (width 0.4064) (layer "F.Cu") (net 1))
 (segment (start 95.601985 115.100293) (end 95.601985 123.974293) (width 0.4064) (layer "F.Cu") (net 1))
 (segment (start 131.825985 115.100293) (end 95.601985 115.100293) (width 0.4064) (layer "F.Cu") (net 1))
 (segment (start 77.821985 114.084293) (end 77.821985 123.974293) (width 0.4064) (layer "F.Cu") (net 8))
 (segment (start 140.461985 126.923493) (end 140.461985 114.084293) (width 0.4064) (layer "F.Cu") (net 8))
 (segment (start 140.654585 120.421093) (end 140.654585 126.923493) (width 0.4064) (layer "F.Cu") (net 8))
 (segment (start 140.461985 114.084293) (end 77.821985 114.084293) (width 0.4064) (layer "F.Cu") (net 8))
 (segment (start 140.654585 126.923493) (end 140.461985 126.923493) (width 0.4064) (layer "F.Cu") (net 8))
 (segment (start 75.281985 113.068293) (end 75.281985 123.974293) (width 0.4064) (layer "F.Cu") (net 6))
 (segment (start 149.351985 126.923493) (end 149.351985 113.068293) (width 0.4064) (layer "F.Cu") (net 6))
 (segment (start 149.351985 113.068293) (end 75.281985 113.068293) (width 0.4064) (layer "F.Cu") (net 6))
 (segment (start 149.346585 126.923493) (end 149.351985 126.923493) (width 0.4064) (layer "F.Cu") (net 6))
 (segment (start 149.346585 120.421093) (end 149.346585 126.923493) (width 0.4064) (layer "F.Cu") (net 6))
 (segment (start 82.901985 97.320293) (end 82.901985 101.114293) (width 0.8128) (layer "F.Cu") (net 2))
 (segment (start 131.317985 97.320293) (end 82.901985 97.320293) (width 0.8128) (layer "F.Cu") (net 2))
 (segment (start 131.465985 88.948293) (end 131.317985 88.948293) (width 0.4064) (layer "F.Cu") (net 2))
 (segment (start 131.317985 88.948293) (end 131.317985 97.320293) (width 0.8128) (layer "F.Cu") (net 2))
 (segment (start 136.133385 120.421093) (end 136.133385 126.923493) (width 0.4064) (layer "B.Cu") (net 2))
 (segment (start 82.803985 112.560293) (end 90.521985 112.560293) (width 0.8128) (layer "B.Cu") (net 2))
 (segment (start 159.257985 92.082293) (end 159.257985 123.736293) (width 0.4064) (layer "B.Cu") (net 2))
 (segment (start 90.423985 123.974293) (end 90.423985 127.292293) (width 0.4064) (layer "B.Cu") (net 2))
 (segment (start 72.741985 123.974293) (end 72.741985 112.560293) (width 0.8128) (layer "B.Cu") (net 2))
 (segment (start 154.519985 92.082293) (end 159.257985 92.082293) (width 0.4064) (layer "B.Cu") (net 2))
 (segment (start 118.871985 123.736293) (end 144.825385 123.736293) (width 0.4064) (layer "B.Cu") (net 2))
 (segment (start 82.803985 101.114293) (end 82.803985 112.560293) (width 0.8128) (layer "B.Cu") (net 2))
 (segment (start 82.901985 101.114293) (end 82.803985 101.114293) (width 0.4064) (layer "B.Cu") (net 2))
 (segment (start 90.423985 127.292293) (end 118.749385 127.292293) (width 0.4064) (layer "B.Cu") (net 2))
 (segment (start 118.749385 120.421093) (end 118.871985 120.421093) (width 0.4064) (layer "B.Cu") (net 2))
 (segment (start 118.749385 127.292293) (end 118.749385 126.923493) (width 0.4064) (layer "B.Cu") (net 2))
 (segment (start 144.825385 123.736293) (end 144.825385 126.923493) (width 0.4064) (layer "B.Cu") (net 2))
 (segment (start 118.749385 126.923493) (end 118.749385 120.421093) (width 0.4064) (layer "B.Cu") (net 2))
 (segment (start 127.441385 120.421093) (end 127.441385 126.923493) (width 0.4064) (layer "B.Cu") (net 2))
 (segment (start 159.257985 123.736293) (end 144.825385 123.736293) (width 0.4064) (layer "B.Cu") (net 2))
 (segment (start 144.825385 123.736293) (end 144.825385 120.421093) (width 0.4064) (layer "B.Cu") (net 2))
 (segment (start 118.871985 120.421093) (end 118.871985 123.736293) (width 0.4064) (layer "B.Cu") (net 2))
 (segment (start 90.521985 123.974293) (end 90.423985 123.974293) (width 0.4064) (layer "B.Cu") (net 2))
 (segment (start 72.741985 112.560293) (end 72.741985 101.114293) (width 0.8128) (layer "B.Cu") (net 2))
 (segment (start 82.803985 112.560293) (end 72.741985 112.560293) (width 0.8128) (layer "B.Cu") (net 2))
 (segment (start 90.521985 112.560293) (end 90.521985 123.974293) (width 0.8128) (layer "B.Cu") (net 2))
 (segment (start 70.201985 88.928293) (end 70.201985 101.114293) (width 0.8128) (layer "F.Cu") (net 9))
 (segment (start 70.209985 88.928293) (end 70.201985 88.928293) (width 0.4064) (layer "F.Cu") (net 9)))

